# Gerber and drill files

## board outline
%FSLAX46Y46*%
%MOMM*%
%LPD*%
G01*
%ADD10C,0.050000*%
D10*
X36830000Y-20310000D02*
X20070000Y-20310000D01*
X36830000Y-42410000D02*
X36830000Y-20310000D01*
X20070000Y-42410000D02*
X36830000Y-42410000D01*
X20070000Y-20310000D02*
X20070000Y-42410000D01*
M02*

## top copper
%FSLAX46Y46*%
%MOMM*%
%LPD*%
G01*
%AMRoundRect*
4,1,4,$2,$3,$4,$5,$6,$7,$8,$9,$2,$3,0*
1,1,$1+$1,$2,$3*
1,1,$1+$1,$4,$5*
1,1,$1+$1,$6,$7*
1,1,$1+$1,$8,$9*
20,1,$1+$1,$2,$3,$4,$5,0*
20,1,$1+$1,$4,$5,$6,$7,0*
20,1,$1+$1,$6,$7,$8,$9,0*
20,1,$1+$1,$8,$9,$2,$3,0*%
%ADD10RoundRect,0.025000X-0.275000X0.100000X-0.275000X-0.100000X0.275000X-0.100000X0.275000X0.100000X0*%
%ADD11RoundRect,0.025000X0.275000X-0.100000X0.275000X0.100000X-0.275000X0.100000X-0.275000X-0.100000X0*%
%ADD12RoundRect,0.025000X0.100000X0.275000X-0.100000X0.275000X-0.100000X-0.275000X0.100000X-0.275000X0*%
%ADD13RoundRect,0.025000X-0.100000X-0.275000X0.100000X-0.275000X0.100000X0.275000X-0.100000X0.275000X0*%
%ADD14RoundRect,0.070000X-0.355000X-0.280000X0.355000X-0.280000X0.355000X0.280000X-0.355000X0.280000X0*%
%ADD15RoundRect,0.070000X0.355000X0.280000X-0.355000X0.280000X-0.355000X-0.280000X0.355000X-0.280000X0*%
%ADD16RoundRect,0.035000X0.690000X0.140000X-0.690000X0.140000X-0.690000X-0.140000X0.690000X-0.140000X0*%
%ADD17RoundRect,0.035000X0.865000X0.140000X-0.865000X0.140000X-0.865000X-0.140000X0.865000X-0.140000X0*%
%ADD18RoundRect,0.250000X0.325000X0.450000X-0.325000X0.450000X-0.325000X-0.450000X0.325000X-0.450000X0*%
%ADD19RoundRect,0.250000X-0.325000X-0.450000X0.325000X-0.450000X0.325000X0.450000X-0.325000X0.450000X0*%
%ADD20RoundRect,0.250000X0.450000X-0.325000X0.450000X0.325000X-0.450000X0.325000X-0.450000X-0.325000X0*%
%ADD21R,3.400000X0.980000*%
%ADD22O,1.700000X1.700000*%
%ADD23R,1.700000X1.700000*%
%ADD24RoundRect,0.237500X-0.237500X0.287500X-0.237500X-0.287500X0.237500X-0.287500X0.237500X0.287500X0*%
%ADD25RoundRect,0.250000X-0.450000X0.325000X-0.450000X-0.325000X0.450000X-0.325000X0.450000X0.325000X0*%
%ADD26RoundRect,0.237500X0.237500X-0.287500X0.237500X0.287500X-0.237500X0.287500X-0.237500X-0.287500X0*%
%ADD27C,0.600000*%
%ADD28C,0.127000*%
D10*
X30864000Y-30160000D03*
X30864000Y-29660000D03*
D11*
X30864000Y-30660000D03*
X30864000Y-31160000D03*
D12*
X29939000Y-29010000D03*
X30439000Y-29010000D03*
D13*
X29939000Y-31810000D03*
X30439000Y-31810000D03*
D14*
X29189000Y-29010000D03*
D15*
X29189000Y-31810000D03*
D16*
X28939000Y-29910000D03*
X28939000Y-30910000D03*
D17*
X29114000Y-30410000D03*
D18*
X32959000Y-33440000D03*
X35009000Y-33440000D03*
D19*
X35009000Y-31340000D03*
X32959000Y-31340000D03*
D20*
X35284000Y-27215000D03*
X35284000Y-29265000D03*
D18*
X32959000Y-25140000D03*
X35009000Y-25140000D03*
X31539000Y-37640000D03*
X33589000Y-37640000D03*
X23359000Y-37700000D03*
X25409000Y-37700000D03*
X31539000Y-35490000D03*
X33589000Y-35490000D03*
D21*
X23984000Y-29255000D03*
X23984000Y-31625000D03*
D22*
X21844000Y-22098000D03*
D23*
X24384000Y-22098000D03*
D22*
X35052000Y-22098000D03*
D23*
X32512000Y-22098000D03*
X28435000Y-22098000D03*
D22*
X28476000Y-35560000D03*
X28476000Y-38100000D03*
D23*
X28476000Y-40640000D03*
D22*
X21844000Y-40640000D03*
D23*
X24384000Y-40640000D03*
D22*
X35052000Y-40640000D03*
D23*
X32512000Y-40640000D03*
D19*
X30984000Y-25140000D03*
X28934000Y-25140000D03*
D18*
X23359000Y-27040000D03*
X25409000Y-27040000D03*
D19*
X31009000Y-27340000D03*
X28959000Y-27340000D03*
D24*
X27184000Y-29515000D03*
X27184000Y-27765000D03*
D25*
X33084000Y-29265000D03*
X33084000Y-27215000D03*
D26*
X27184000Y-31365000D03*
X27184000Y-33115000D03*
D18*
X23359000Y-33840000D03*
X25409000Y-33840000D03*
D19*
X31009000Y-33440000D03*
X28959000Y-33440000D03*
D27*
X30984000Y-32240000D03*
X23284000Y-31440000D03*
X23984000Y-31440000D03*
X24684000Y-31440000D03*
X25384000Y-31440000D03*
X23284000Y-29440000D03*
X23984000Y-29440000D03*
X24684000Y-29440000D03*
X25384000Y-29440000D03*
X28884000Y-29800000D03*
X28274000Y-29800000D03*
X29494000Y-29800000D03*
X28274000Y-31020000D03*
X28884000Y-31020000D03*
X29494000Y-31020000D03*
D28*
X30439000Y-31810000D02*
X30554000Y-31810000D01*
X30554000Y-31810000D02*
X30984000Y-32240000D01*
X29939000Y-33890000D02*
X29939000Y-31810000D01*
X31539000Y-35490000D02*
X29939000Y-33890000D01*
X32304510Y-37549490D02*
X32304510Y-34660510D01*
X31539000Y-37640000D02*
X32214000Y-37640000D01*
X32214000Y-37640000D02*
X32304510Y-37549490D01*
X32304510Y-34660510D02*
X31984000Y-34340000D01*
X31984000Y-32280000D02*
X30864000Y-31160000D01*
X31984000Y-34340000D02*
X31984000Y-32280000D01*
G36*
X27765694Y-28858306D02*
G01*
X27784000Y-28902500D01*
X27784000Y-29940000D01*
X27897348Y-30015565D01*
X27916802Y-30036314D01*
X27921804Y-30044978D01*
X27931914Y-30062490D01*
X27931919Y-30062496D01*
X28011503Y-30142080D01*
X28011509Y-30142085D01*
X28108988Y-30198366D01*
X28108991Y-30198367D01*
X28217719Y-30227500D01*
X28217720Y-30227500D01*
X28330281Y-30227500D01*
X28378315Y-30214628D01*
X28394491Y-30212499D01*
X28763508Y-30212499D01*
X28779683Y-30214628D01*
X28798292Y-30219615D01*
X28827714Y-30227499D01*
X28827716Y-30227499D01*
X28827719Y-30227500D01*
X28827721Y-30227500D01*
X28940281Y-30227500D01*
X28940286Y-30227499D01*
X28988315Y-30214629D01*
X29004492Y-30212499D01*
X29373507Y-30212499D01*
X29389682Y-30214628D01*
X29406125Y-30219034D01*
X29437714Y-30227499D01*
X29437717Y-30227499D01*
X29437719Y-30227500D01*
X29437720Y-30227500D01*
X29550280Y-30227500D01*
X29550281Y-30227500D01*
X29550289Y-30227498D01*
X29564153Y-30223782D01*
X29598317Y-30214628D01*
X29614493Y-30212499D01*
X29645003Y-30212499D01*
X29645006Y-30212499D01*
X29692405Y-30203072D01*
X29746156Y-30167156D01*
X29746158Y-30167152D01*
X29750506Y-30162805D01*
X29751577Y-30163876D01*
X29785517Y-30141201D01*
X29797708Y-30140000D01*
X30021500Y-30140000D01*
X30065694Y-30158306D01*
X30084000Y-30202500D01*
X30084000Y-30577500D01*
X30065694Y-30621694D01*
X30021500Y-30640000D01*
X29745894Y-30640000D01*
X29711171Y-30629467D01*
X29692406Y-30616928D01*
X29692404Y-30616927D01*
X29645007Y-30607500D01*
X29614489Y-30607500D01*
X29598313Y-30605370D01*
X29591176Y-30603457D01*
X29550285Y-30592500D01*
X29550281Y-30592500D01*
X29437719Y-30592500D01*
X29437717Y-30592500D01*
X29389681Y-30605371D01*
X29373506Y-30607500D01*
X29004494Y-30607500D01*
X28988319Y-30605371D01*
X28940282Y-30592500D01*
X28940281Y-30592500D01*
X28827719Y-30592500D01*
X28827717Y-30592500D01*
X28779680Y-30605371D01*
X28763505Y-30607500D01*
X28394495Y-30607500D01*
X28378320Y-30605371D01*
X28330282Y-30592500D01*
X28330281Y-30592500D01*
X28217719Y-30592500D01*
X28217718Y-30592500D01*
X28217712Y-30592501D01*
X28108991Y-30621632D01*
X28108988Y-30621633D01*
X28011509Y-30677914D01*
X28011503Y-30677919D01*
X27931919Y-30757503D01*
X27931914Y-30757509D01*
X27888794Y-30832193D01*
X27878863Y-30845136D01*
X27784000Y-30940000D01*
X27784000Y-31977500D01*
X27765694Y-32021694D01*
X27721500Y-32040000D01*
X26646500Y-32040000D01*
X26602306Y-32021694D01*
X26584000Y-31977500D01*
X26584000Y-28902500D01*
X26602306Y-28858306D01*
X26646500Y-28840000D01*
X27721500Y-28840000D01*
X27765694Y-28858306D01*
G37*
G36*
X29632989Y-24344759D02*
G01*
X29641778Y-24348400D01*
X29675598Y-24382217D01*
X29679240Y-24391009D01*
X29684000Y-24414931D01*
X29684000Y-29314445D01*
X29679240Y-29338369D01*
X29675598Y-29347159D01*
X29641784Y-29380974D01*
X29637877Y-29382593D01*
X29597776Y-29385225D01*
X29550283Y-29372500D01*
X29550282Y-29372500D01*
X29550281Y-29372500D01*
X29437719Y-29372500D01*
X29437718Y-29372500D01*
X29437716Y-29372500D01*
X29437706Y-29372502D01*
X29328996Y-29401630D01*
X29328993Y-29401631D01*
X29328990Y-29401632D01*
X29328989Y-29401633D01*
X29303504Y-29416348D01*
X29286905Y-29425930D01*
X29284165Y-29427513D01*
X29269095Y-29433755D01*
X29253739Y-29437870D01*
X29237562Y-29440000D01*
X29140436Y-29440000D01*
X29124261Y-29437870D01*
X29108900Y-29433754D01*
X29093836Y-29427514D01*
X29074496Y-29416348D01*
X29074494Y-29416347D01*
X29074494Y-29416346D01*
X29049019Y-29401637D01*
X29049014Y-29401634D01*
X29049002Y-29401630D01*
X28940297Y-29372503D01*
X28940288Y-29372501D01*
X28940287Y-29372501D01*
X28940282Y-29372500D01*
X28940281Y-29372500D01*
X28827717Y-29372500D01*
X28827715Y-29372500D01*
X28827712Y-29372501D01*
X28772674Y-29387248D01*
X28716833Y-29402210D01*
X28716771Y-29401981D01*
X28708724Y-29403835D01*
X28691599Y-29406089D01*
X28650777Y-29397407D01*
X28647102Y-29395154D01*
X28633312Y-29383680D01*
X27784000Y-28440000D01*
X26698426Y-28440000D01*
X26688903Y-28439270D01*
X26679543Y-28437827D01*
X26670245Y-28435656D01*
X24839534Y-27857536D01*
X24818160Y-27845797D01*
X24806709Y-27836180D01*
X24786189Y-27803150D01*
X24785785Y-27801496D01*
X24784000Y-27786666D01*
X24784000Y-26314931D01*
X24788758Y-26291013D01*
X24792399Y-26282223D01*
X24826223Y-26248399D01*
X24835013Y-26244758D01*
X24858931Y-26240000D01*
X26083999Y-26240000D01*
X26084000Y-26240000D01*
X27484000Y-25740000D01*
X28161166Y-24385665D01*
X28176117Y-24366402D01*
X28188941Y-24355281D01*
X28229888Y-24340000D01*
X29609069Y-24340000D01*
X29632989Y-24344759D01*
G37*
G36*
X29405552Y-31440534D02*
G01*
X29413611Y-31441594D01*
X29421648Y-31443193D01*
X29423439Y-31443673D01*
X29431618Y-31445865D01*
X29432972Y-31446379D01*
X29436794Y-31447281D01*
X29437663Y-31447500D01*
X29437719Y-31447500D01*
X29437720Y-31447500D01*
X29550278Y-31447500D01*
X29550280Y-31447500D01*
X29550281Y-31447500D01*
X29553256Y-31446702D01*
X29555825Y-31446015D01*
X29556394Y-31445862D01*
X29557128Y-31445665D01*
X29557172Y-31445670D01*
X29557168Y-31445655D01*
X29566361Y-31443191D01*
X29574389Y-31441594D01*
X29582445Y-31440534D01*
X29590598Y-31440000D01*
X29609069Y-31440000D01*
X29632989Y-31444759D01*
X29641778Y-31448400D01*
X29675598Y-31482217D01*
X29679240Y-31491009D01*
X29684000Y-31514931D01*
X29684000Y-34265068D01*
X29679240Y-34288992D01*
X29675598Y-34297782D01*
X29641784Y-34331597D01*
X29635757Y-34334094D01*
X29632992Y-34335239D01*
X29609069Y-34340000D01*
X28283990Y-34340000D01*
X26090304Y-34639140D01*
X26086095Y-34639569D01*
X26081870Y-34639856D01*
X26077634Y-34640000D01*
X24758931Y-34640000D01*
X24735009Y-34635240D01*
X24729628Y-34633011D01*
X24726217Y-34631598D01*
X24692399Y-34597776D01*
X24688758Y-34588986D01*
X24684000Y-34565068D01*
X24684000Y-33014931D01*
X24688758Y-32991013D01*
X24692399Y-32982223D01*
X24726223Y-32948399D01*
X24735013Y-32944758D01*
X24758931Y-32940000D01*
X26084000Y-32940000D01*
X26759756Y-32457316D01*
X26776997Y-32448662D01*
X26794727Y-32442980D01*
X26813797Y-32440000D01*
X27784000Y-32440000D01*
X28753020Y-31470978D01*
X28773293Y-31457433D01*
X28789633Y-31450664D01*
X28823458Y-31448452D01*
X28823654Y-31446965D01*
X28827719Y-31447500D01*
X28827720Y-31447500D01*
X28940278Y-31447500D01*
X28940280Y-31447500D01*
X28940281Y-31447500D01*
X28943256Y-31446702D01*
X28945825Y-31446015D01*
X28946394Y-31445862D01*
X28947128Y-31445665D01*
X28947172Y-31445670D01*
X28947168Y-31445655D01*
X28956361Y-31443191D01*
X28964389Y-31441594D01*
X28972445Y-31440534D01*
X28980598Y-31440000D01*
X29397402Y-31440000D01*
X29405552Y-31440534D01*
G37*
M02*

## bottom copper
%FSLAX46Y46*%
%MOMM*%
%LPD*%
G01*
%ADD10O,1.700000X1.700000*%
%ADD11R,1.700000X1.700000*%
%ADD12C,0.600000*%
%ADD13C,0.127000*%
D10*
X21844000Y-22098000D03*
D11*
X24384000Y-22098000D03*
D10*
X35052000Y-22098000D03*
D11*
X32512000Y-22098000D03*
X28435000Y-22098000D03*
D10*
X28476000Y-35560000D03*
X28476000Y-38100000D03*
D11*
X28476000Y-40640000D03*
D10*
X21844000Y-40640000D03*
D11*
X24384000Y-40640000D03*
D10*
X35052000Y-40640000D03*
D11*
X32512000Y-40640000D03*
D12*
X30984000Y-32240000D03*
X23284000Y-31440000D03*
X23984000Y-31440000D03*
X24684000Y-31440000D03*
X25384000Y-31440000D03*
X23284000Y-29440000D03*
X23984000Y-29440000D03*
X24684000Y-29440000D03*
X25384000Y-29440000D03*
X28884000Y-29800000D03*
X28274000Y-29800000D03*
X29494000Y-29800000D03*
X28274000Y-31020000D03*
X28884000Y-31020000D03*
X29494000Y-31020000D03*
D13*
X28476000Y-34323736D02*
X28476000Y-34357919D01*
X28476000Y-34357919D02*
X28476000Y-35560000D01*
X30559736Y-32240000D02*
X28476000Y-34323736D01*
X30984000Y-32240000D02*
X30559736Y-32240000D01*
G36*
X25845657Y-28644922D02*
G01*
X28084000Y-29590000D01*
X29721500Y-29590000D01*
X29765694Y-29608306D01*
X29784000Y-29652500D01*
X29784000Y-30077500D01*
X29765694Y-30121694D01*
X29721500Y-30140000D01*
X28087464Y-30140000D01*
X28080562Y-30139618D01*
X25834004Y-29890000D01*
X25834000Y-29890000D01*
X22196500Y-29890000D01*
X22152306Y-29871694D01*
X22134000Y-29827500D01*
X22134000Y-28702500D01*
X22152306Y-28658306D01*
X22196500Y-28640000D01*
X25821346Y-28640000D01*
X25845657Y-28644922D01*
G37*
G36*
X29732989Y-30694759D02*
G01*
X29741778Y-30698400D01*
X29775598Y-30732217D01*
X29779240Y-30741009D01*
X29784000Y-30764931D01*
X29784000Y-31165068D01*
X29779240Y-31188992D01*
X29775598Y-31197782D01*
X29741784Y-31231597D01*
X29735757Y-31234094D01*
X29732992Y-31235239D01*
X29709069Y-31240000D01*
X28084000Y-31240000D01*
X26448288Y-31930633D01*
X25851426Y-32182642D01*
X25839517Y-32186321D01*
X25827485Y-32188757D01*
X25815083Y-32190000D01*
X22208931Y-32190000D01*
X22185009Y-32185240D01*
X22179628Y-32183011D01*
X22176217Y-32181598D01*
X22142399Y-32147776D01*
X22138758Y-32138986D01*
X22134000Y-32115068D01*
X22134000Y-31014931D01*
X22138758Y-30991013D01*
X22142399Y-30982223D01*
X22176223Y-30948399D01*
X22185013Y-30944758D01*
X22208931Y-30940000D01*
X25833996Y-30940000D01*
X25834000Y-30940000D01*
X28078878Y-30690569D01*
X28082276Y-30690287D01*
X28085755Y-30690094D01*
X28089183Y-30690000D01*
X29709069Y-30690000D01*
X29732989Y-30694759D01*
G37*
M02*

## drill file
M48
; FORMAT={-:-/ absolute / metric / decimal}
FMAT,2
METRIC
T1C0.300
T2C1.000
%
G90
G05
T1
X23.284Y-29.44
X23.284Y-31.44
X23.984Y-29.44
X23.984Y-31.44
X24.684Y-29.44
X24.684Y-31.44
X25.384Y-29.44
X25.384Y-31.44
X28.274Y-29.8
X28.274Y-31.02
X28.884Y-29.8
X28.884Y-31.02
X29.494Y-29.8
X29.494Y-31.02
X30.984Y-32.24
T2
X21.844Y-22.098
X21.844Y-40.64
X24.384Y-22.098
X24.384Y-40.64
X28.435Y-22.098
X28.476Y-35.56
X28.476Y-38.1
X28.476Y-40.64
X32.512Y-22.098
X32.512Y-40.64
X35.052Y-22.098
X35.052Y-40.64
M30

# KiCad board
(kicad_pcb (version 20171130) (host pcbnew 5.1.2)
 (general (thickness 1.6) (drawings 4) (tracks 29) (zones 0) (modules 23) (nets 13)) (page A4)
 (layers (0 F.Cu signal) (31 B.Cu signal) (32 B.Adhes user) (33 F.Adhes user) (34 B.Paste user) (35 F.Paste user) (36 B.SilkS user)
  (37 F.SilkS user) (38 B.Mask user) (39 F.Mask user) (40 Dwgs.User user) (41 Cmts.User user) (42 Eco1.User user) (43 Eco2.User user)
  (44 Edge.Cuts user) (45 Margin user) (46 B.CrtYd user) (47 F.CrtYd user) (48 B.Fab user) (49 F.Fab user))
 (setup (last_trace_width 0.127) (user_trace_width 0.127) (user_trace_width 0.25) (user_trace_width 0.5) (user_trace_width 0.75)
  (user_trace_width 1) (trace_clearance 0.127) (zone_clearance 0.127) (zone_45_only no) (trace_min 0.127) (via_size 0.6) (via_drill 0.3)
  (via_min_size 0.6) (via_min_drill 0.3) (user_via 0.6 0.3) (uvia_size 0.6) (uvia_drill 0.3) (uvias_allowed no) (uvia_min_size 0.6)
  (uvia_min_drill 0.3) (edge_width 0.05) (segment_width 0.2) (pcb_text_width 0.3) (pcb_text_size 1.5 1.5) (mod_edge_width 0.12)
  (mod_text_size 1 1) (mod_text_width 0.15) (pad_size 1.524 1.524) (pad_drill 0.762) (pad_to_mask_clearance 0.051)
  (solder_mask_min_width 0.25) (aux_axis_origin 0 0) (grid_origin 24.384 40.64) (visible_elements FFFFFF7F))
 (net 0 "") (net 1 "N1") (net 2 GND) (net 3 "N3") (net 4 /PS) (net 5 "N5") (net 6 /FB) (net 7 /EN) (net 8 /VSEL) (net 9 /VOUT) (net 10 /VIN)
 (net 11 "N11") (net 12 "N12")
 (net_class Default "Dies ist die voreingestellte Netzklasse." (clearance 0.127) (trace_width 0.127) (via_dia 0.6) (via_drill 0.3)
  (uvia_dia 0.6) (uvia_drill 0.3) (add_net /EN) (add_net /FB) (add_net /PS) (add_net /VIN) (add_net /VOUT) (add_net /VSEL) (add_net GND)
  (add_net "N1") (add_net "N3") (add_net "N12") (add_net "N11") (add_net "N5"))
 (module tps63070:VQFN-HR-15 (layer F.Cu) (at 29.714 30.41 180)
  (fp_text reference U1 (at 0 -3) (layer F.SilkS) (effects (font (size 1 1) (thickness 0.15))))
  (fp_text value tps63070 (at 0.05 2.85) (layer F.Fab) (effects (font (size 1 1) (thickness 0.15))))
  (pad "" smd roundrect (at 1.06 0 270) (size 0.25 0.72) (layers F.Paste) (roundrect_rratio 0.1))
  (pad "" smd roundrect (at 0.14 0 270) (size 0.25 0.72) (layers F.Paste) (roundrect_rratio 0.1))
  (pad "" smd roundrect (at 1.163 0.5 270) (size 0.25 0.575) (layers F.Paste) (roundrect_rratio 0.1))
  (pad "" smd roundrect (at 0.388 0.5 270) (size 0.25 0.575) (layers F.Paste) (roundrect_rratio 0.1))
  (pad "" smd roundrect (at 1.163 -0.5 270) (size 0.25 0.575) (layers F.Paste) (roundrect_rratio 0.1))
  (pad "" smd roundrect (at 0.388 -0.5 270) (size 0.25 0.575) (layers F.Paste) (roundrect_rratio 0.1))
  (pad 3 smd roundrect (at -1.15 0.25 270) (size 0.25 0.6) (layers F.Cu F.Paste F.Mask) (roundrect_rratio 0.1) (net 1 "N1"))
  (pad 4 smd roundrect (at -1.15 0.75 270) (size 0.25 0.6) (layers F.Cu F.Paste F.Mask) (roundrect_rratio 0.1) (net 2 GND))
  (pad 2 smd roundrect (at -1.15 -0.25 90) (size 0.25 0.6) (layers F.Cu F.Paste F.Mask) (roundrect_rratio 0.1) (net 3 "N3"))
  (pad 1 smd roundrect (at -1.15 -0.75 90) (size 0.25 0.6) (layers F.Cu F.Paste F.Mask) (roundrect_rratio 0.1) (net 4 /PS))
  (pad 6 smd roundrect (at -0.225 1.4 180) (size 0.25 0.6) (layers F.Cu F.Paste F.Mask) (roundrect_rratio 0.1) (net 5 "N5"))
  (pad 5 smd roundrect (at -0.725 1.4 180) (size 0.25 0.6) (layers F.Cu F.Paste F.Mask) (roundrect_rratio 0.1) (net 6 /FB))
  (pad 14 smd roundrect (at -0.225 -1.4) (size 0.25 0.6) (layers F.Cu F.Paste F.Mask) (roundrect_rratio 0.1) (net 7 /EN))
  (pad 15 smd roundrect (at -0.725 -1.4) (size 0.25 0.6) (layers F.Cu F.Paste F.Mask) (roundrect_rratio 0.1) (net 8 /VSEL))
  (pad 7 smd roundrect (at 0.525 1.4) (size 0.85 0.7) (layers F.Cu) (roundrect_rratio 0.1) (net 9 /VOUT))
  (pad 12 smd roundrect (at 0.525 -1.4 180) (size 0.85 0.7) (layers F.Cu) (roundrect_rratio 0.1) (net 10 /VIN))
  (pad "" smd roundrect (at 0.775 0.5 180) (size 1.35 0.25) (layers F.Mask) (roundrect_rratio 0.1))
  (pad 9 smd roundrect (at 0.775 0.5 180) (size 1.45 0.35) (layers F.Cu) (roundrect_rratio 0.1) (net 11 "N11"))
  (pad "" smd roundrect (at 0.775 -0.5 180) (size 1.35 0.25) (layers F.Mask) (roundrect_rratio 0.1))
  (pad 11 smd roundrect (at 0.775 -0.5 180) (size 1.45 0.35) (layers F.Cu) (roundrect_rratio 0.1) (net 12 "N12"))
  (pad "" smd roundrect (at 0.6 0 180) (size 1.7 0.25) (layers F.Mask) (roundrect_rratio 0.1))
  (pad 10 smd roundrect (at 0.6 0 180) (size 1.8 0.35) (layers F.Cu) (roundrect_rratio 0.1) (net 2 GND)))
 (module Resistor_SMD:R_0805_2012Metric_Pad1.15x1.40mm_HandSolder (layer F.Cu) (at 33.984 33.44 180)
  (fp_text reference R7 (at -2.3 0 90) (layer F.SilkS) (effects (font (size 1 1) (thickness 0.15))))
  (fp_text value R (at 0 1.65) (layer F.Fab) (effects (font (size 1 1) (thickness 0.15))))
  (pad 2 smd roundrect (at 1.025 0 180) (size 1.15 1.4) (layers F.Cu F.Paste F.Mask) (roundrect_rratio 0.217391) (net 3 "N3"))
  (pad 1 smd roundrect (at -1.025 0 180) (size 1.15 1.4) (layers F.Cu F.Paste F.Mask) (roundrect_rratio 0.217391) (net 9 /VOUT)))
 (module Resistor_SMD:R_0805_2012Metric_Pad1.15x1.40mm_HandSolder (layer F.Cu) (at 33.984 31.34)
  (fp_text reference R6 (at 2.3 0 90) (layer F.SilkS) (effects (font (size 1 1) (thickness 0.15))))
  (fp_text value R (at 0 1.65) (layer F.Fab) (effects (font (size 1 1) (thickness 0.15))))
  (pad 2 smd roundrect (at 1.025 0) (size 1.15 1.4) (layers F.Cu F.Paste F.Mask) (roundrect_rratio 0.217391) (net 2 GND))
  (pad 1 smd roundrect (at -1.025 0) (size 1.15 1.4) (layers F.Cu F.Paste F.Mask) (roundrect_rratio 0.217391) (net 6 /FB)))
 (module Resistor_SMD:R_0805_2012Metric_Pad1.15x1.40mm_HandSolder (layer F.Cu) (at 35.284 28.24 90)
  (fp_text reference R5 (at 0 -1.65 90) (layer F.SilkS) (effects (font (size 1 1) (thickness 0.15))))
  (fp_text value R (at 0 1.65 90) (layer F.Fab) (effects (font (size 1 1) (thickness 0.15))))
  (pad 2 smd roundrect (at 1.025 0 90) (size 1.15 1.4) (layers F.Cu F.Paste F.Mask) (roundrect_rratio 0.217391) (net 6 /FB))
  (pad 1 smd roundrect (at -1.025 0 90) (size 1.15 1.4) (layers F.Cu F.Paste F.Mask) (roundrect_rratio 0.217391) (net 9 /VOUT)))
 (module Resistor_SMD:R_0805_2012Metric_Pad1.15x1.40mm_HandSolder (layer F.Cu) (at 33.984 25.14 180)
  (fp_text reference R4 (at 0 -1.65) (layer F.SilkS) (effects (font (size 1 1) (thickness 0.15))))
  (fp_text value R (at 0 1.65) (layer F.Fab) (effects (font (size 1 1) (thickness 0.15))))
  (pad 2 smd roundrect (at 1.025 0 180) (size 1.15 1.4) (layers F.Cu F.Paste F.Mask) (roundrect_rratio 0.217391) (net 5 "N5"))
  (pad 1 smd roundrect (at -1.025 0 180) (size 1.15 1.4) (layers F.Cu F.Paste F.Mask) (roundrect_rratio 0.217391) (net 6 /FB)))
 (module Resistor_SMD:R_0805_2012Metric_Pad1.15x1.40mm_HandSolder (layer F.Cu) (at 32.564 37.64 180)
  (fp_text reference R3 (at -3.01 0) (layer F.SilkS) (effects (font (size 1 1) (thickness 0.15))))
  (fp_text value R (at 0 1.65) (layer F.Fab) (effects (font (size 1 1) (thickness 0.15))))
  (pad 2 smd roundrect (at 1.025 0 180) (size 1.15 1.4) (layers F.Cu F.Paste F.Mask) (roundrect_rratio 0.217391) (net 4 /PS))
  (pad 1 smd roundrect (at -1.025 0 180) (size 1.15 1.4) (layers F.Cu F.Paste F.Mask) (roundrect_rratio 0.217391) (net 10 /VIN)))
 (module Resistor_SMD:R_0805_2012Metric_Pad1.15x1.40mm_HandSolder (layer F.Cu) (at 24.384 37.7 180)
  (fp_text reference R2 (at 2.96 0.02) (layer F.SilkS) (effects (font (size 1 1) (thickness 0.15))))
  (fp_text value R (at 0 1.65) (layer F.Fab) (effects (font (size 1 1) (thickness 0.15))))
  (pad 2 smd roundrect (at 1.025 0 180) (size 1.15 1.4) (layers F.Cu F.Paste F.Mask) (roundrect_rratio 0.217391) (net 2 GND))
  (pad 1 smd roundrect (at -1.025 0 180) (size 1.15 1.4) (layers F.Cu F.Paste F.Mask) (roundrect_rratio 0.217391) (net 8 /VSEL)))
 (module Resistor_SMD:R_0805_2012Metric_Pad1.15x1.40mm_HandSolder (layer F.Cu) (at 32.564 35.49 180)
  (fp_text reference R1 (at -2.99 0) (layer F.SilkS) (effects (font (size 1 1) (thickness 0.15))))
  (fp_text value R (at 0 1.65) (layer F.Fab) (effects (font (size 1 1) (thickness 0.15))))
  (pad 2 smd roundrect (at 1.025 0 180) (size 1.15 1.4) (layers F.Cu F.Paste F.Mask) (roundrect_rratio 0.217391) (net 7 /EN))
  (pad 1 smd roundrect (at -1.025 0 180) (size 1.15 1.4) (layers F.Cu F.Paste F.Mask) (roundrect_rratio 0.217391) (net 10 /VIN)))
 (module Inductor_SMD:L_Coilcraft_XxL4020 (layer F.Cu) (at 23.984 30.44 90)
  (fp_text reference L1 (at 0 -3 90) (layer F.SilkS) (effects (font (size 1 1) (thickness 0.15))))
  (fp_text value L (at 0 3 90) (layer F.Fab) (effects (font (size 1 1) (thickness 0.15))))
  (pad 2 smd rect (at 1.185 0 90) (size 0.98 3.4) (layers F.Cu F.Paste F.Mask) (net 11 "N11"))
  (pad 1 smd rect (at -1.185 0 90) (size 0.98 3.4) (layers F.Cu F.Paste F.Mask) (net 12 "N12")))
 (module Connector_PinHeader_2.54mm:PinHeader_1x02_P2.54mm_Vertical (layer B.Cu) (at 24.384 22.098 90)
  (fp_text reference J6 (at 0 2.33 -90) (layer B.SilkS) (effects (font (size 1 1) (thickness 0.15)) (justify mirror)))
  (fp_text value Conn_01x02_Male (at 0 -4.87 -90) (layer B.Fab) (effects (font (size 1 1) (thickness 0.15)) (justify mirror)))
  (pad 2 thru_hole oval (at 0 -2.54 90) (size 1.7 1.7) (drill 1) (layers *.Cu *.Mask) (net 2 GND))
  (pad 1 thru_hole rect (at 0 0 90) (size 1.7 1.7) (drill 1) (layers *.Cu *.Mask) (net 2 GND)))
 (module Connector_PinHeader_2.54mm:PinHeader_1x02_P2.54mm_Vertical (layer B.Cu) (at 32.512 22.098 270)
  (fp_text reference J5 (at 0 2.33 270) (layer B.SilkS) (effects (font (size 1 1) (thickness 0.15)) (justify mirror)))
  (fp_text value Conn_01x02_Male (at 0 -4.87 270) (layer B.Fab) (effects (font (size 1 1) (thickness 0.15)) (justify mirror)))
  (pad 2 thru_hole oval (at 0 -2.54 270) (size 1.7 1.7) (drill 1) (layers *.Cu *.Mask) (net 9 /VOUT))
  (pad 1 thru_hole rect (at 0 0 270) (size 1.7 1.7) (drill 1) (layers *.Cu *.Mask) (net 9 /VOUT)))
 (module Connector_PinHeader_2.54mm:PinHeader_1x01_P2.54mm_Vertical (layer B.Cu) (at 28.435 22.098)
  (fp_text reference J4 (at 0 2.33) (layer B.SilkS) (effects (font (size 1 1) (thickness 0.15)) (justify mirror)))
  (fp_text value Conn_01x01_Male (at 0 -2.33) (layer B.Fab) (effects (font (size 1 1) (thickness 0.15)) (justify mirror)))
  (pad 1 thru_hole rect (at 0 0) (size 1.7 1.7) (drill 1) (layers *.Cu *.Mask) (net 3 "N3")))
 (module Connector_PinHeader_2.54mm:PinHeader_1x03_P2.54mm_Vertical (layer B.Cu) (at 28.476 40.64)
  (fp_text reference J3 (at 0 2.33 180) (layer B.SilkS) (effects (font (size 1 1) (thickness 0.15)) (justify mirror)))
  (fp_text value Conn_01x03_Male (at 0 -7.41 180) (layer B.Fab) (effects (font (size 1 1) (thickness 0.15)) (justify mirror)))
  (pad 3 thru_hole oval (at 0 -5.08) (size 1.7 1.7) (drill 1) (layers *.Cu *.Mask) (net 8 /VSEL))
  (pad 2 thru_hole oval (at 0 -2.54) (size 1.7 1.7) (drill 1) (layers *.Cu *.Mask) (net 7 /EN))
  (pad 1 thru_hole rect (at 0 0) (size 1.7 1.7) (drill 1) (layers *.Cu *.Mask) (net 4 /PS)))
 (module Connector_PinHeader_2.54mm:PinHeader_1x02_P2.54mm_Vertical (layer B.Cu) (at 24.384 40.64 90)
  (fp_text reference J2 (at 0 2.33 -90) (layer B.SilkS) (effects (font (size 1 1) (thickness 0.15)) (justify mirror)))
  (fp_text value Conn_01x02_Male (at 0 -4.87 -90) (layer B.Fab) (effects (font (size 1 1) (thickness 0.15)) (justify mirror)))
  (pad 2 thru_hole oval (at 0 -2.54 90) (size 1.7 1.7) (drill 1) (layers *.Cu *.Mask) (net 2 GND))
  (pad 1 thru_hole rect (at 0 0 90) (size 1.7 1.7) (drill 1) (layers *.Cu *.Mask) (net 2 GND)))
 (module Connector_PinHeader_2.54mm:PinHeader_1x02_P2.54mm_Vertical (layer B.Cu) (at 32.512 40.64 270)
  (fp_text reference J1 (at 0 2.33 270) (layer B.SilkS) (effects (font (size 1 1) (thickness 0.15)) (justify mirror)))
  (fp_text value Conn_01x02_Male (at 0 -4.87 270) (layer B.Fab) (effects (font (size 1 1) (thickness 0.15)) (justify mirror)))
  (pad 2 thru_hole oval (at 0 -2.54 270) (size 1.7 1.7) (drill 1) (layers *.Cu *.Mask) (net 10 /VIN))
  (pad 1 thru_hole rect (at 0 0 270) (size 1.7 1.7) (drill 1) (layers *.Cu *.Mask) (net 10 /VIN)))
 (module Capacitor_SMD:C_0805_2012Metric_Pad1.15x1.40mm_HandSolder (layer F.Cu) (at 29.959 25.14)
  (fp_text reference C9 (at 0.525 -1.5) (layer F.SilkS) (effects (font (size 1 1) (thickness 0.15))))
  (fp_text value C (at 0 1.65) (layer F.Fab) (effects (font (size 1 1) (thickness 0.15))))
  (pad 2 smd roundrect (at 1.025 0) (size 1.15 1.4) (layers F.Cu F.Paste F.Mask) (roundrect_rratio 0.217391) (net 2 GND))
  (pad 1 smd roundrect (at -1.025 0) (size 1.15 1.4) (layers F.Cu F.Paste F.Mask) (roundrect_rratio 0.217391) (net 9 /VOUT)))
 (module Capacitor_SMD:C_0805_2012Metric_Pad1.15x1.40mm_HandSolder (layer F.Cu) (at 24.384 27.04 180)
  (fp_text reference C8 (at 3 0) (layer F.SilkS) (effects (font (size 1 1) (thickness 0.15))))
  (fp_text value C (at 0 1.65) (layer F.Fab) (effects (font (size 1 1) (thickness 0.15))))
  (pad 2 smd roundrect (at 1.025 0 180) (size 1.15 1.4) (layers F.Cu F.Paste F.Mask) (roundrect_rratio 0.217391) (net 2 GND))
  (pad 1 smd roundrect (at -1.025 0 180) (size 1.15 1.4) (layers F.Cu F.Paste F.Mask) (roundrect_rratio 0.217391) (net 9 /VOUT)))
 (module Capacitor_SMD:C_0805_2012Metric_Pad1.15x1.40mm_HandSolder (layer F.Cu) (at 29.984 27.34)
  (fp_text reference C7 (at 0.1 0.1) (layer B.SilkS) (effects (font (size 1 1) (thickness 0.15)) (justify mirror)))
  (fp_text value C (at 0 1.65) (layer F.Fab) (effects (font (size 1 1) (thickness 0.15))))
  (pad 2 smd roundrect (at 1.025 0) (size 1.15 1.4) (layers F.Cu F.Paste F.Mask) (roundrect_rratio 0.217391) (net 2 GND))
  (pad 1 smd roundrect (at -1.025 0) (size 1.15 1.4) (layers F.Cu F.Paste F.Mask) (roundrect_rratio 0.217391) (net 9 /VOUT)))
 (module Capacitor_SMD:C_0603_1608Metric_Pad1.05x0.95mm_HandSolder (layer F.Cu) (at 27.184 28.64 270)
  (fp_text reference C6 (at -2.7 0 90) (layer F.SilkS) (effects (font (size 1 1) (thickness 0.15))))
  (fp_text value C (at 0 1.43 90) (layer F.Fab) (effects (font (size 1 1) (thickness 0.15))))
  (pad 2 smd roundrect (at 0.875 0 270) (size 1.05 0.95) (layers F.Cu F.Paste F.Mask) (roundrect_rratio 0.25) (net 2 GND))
  (pad 1 smd roundrect (at -0.875 0 270) (size 1.05 0.95) (layers F.Cu F.Paste F.Mask) (roundrect_rratio 0.25) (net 9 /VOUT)))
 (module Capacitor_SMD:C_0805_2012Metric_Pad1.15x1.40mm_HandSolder (layer F.Cu) (at 33.084 28.24 270)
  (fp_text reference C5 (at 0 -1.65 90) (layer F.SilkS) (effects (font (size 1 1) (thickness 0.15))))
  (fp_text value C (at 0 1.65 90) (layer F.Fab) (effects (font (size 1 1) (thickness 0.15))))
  (pad 2 smd roundrect (at 1.025 0 270) (size 1.15 1.4) (layers F.Cu F.Paste F.Mask) (roundrect_rratio 0.217391) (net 1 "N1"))
  (pad 1 smd roundrect (at -1.025 0 270) (size 1.15 1.4) (layers F.Cu F.Paste F.Mask) (roundrect_rratio 0.217391) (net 2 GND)))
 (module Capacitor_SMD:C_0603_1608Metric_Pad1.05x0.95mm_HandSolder (layer F.Cu) (at 27.184 32.24 90)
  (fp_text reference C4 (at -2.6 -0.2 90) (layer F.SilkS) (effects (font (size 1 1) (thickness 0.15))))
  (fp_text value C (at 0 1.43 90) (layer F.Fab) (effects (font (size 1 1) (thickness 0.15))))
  (pad 2 smd roundrect (at 0.875 0 90) (size 1.05 0.95) (layers F.Cu F.Paste F.Mask) (roundrect_rratio 0.25) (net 2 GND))
  (pad 1 smd roundrect (at -0.875 0 90) (size 1.05 0.95) (layers F.Cu F.Paste F.Mask) (roundrect_rratio 0.25) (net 10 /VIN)))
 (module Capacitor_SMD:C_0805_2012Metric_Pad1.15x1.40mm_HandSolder (layer F.Cu) (at 24.384 33.84 180)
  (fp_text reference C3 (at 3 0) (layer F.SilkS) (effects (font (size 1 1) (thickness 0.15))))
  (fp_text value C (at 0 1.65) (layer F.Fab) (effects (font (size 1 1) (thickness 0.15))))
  (pad 2 smd roundrect (at 1.025 0 180) (size 1.15 1.4) (layers F.Cu F.Paste F.Mask) (roundrect_rratio 0.217391) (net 2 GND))
  (pad 1 smd roundrect (at -1.025 0 180) (size 1.15 1.4) (layers F.Cu F.Paste F.Mask) (roundrect_rratio 0.217391) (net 10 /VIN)))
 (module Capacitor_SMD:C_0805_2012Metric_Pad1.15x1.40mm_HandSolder (layer F.Cu) (at 29.984 33.44)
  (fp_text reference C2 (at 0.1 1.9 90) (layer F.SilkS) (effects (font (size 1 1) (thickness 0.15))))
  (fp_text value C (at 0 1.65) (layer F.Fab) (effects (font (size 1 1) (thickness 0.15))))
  (pad 2 smd roundrect (at 1.025 0) (size 1.15 1.4) (layers F.Cu F.Paste F.Mask) (roundrect_rratio 0.217391) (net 2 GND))
  (pad 1 smd roundrect (at -1.025 0) (size 1.15 1.4) (layers F.Cu F.Paste F.Mask) (roundrect_rratio 0.217391) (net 10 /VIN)))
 (gr_line (start 36.83 20.31) (end 20.07 20.31) (layer Edge.Cuts) (width 0.05))
 (gr_line (start 36.83 42.41) (end 36.83 20.31) (layer Edge.Cuts) (width 0.05))
 (gr_line (start 20.07 42.41) (end 36.83 42.41) (layer Edge.Cuts) (width 0.05))
 (gr_line (start 20.07 20.31) (end 20.07 42.41) (layer Edge.Cuts) (width 0.05))
 (via (at 30.984 32.24) (size 0.6) (drill 0.3) (layers F.Cu B.Cu) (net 8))
 (segment (start 30.439 31.81) (end 30.554 31.81) (width 0.127) (layer F.Cu) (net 8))
 (segment (start 30.554 31.81) (end 30.984 32.24) (width 0.127) (layer F.Cu) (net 8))
 (segment (start 28.476 34.323736) (end 28.476 34.357919) (width 0.127) (layer B.Cu) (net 8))
 (segment (start 28.476 34.357919) (end 28.476 35.56) (width 0.127) (layer B.Cu) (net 8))
 (segment (start 30.559736 32.24) (end 28.476 34.323736) (width 0.127) (layer B.Cu) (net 8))
 (segment (start 30.984 32.24) (end 30.559736 32.24) (width 0.127) (layer B.Cu) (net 8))
 (segment (start 29.939 33.89) (end 29.939 31.81) (width 0.127) (layer F.Cu) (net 7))
 (segment (start 31.539 35.49) (end 29.939 33.89) (width 0.127) (layer F.Cu) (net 7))
 (segment (start 32.30451 37.54949) (end 32.30451 34.66051) (width 0.127) (layer F.Cu) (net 4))
 (segment (start 31.539 37.64) (end 32.214 37.64) (width 0.127) (layer F.Cu) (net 4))
 (segment (start 32.214 37.64) (end 32.30451 37.54949) (width 0.127) (layer F.Cu) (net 4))
 (segment (start 32.30451 34.66051) (end 31.984 34.34) (width 0.127) (layer F.Cu) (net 4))
 (segment (start 31.984 32.28) (end 30.864 31.16) (width 0.127) (layer F.Cu) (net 4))
 (segment (start 31.984 34.34) (end 31.984 32.28) (width 0.127) (layer F.Cu) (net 4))
 (via (at 23.284 31.44) (size 0.6) (drill 0.3) (layers F.Cu B.Cu) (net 12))
 (via (at 23.984 31.44) (size 0.6) (drill 0.3) (layers F.Cu B.Cu) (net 12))
 (via (at 24.684 31.44) (size 0.6) (drill 0.3) (layers F.Cu B.Cu) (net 12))
 (via (at 25.384 31.44) (size 0.6) (drill 0.3) (layers F.Cu B.Cu) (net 12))
 (via (at 23.284 29.44) (size 0.6) (drill 0.3) (layers F.Cu B.Cu) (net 11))
 (via (at 23.984 29.44) (size 0.6) (drill 0.3) (layers F.Cu B.Cu) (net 11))
 (via (at 24.684 29.44) (size 0.6) (drill 0.3) (layers F.Cu B.Cu) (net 11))
 (via (at 25.384 29.44) (size 0.6) (drill 0.3) (layers F.Cu B.Cu) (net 11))
 (via (at 28.884 29.8) (size 0.6) (drill 0.3) (layers F.Cu B.Cu) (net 11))
 (via (at 28.274 29.8) (size 0.6) (drill 0.3) (layers F.Cu B.Cu) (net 11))
 (via (at 29.494 29.8) (size 0.6) (drill 0.3) (layers F.Cu B.Cu) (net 11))
 (via (at 28.274 31.02) (size 0.6) (drill 0.3) (layers F.Cu B.Cu) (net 12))
 (via (at 28.884 31.02) (size 0.6) (drill 0.3) (layers F.Cu B.Cu) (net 12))
 (via (at 29.494 31.02) (size 0.6) (drill 0.3) (layers F.Cu B.Cu) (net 12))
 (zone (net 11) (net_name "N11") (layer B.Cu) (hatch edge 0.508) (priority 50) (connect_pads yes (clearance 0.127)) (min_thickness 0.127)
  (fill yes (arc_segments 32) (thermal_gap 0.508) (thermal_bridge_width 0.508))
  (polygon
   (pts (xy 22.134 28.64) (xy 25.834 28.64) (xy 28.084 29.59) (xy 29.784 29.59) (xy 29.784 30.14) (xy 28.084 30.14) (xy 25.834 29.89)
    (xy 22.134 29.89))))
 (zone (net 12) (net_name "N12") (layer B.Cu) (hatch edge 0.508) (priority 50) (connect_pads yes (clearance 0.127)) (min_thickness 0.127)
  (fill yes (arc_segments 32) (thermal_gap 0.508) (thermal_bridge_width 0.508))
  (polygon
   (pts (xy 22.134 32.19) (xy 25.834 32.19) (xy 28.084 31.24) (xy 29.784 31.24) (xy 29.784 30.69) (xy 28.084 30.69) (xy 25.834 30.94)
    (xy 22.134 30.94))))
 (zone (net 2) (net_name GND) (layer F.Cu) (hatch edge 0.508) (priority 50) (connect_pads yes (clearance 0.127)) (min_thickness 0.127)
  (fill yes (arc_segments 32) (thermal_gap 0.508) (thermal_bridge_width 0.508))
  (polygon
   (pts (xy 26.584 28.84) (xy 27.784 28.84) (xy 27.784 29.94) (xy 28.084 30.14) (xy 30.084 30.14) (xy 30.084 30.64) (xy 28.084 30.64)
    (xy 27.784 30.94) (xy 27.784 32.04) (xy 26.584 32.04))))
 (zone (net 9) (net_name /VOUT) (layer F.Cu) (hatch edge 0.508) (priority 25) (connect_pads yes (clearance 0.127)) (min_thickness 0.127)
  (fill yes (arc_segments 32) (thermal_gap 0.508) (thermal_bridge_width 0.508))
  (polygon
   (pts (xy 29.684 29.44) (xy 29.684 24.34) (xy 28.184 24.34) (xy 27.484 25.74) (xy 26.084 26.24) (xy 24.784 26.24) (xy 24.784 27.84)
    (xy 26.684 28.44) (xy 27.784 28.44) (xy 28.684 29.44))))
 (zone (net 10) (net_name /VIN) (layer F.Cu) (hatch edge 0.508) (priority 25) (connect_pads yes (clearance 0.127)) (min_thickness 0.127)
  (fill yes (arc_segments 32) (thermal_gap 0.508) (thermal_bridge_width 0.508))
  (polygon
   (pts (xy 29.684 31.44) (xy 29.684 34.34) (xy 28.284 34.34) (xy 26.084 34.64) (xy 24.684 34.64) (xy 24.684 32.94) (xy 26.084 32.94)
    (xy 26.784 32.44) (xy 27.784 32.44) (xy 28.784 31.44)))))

